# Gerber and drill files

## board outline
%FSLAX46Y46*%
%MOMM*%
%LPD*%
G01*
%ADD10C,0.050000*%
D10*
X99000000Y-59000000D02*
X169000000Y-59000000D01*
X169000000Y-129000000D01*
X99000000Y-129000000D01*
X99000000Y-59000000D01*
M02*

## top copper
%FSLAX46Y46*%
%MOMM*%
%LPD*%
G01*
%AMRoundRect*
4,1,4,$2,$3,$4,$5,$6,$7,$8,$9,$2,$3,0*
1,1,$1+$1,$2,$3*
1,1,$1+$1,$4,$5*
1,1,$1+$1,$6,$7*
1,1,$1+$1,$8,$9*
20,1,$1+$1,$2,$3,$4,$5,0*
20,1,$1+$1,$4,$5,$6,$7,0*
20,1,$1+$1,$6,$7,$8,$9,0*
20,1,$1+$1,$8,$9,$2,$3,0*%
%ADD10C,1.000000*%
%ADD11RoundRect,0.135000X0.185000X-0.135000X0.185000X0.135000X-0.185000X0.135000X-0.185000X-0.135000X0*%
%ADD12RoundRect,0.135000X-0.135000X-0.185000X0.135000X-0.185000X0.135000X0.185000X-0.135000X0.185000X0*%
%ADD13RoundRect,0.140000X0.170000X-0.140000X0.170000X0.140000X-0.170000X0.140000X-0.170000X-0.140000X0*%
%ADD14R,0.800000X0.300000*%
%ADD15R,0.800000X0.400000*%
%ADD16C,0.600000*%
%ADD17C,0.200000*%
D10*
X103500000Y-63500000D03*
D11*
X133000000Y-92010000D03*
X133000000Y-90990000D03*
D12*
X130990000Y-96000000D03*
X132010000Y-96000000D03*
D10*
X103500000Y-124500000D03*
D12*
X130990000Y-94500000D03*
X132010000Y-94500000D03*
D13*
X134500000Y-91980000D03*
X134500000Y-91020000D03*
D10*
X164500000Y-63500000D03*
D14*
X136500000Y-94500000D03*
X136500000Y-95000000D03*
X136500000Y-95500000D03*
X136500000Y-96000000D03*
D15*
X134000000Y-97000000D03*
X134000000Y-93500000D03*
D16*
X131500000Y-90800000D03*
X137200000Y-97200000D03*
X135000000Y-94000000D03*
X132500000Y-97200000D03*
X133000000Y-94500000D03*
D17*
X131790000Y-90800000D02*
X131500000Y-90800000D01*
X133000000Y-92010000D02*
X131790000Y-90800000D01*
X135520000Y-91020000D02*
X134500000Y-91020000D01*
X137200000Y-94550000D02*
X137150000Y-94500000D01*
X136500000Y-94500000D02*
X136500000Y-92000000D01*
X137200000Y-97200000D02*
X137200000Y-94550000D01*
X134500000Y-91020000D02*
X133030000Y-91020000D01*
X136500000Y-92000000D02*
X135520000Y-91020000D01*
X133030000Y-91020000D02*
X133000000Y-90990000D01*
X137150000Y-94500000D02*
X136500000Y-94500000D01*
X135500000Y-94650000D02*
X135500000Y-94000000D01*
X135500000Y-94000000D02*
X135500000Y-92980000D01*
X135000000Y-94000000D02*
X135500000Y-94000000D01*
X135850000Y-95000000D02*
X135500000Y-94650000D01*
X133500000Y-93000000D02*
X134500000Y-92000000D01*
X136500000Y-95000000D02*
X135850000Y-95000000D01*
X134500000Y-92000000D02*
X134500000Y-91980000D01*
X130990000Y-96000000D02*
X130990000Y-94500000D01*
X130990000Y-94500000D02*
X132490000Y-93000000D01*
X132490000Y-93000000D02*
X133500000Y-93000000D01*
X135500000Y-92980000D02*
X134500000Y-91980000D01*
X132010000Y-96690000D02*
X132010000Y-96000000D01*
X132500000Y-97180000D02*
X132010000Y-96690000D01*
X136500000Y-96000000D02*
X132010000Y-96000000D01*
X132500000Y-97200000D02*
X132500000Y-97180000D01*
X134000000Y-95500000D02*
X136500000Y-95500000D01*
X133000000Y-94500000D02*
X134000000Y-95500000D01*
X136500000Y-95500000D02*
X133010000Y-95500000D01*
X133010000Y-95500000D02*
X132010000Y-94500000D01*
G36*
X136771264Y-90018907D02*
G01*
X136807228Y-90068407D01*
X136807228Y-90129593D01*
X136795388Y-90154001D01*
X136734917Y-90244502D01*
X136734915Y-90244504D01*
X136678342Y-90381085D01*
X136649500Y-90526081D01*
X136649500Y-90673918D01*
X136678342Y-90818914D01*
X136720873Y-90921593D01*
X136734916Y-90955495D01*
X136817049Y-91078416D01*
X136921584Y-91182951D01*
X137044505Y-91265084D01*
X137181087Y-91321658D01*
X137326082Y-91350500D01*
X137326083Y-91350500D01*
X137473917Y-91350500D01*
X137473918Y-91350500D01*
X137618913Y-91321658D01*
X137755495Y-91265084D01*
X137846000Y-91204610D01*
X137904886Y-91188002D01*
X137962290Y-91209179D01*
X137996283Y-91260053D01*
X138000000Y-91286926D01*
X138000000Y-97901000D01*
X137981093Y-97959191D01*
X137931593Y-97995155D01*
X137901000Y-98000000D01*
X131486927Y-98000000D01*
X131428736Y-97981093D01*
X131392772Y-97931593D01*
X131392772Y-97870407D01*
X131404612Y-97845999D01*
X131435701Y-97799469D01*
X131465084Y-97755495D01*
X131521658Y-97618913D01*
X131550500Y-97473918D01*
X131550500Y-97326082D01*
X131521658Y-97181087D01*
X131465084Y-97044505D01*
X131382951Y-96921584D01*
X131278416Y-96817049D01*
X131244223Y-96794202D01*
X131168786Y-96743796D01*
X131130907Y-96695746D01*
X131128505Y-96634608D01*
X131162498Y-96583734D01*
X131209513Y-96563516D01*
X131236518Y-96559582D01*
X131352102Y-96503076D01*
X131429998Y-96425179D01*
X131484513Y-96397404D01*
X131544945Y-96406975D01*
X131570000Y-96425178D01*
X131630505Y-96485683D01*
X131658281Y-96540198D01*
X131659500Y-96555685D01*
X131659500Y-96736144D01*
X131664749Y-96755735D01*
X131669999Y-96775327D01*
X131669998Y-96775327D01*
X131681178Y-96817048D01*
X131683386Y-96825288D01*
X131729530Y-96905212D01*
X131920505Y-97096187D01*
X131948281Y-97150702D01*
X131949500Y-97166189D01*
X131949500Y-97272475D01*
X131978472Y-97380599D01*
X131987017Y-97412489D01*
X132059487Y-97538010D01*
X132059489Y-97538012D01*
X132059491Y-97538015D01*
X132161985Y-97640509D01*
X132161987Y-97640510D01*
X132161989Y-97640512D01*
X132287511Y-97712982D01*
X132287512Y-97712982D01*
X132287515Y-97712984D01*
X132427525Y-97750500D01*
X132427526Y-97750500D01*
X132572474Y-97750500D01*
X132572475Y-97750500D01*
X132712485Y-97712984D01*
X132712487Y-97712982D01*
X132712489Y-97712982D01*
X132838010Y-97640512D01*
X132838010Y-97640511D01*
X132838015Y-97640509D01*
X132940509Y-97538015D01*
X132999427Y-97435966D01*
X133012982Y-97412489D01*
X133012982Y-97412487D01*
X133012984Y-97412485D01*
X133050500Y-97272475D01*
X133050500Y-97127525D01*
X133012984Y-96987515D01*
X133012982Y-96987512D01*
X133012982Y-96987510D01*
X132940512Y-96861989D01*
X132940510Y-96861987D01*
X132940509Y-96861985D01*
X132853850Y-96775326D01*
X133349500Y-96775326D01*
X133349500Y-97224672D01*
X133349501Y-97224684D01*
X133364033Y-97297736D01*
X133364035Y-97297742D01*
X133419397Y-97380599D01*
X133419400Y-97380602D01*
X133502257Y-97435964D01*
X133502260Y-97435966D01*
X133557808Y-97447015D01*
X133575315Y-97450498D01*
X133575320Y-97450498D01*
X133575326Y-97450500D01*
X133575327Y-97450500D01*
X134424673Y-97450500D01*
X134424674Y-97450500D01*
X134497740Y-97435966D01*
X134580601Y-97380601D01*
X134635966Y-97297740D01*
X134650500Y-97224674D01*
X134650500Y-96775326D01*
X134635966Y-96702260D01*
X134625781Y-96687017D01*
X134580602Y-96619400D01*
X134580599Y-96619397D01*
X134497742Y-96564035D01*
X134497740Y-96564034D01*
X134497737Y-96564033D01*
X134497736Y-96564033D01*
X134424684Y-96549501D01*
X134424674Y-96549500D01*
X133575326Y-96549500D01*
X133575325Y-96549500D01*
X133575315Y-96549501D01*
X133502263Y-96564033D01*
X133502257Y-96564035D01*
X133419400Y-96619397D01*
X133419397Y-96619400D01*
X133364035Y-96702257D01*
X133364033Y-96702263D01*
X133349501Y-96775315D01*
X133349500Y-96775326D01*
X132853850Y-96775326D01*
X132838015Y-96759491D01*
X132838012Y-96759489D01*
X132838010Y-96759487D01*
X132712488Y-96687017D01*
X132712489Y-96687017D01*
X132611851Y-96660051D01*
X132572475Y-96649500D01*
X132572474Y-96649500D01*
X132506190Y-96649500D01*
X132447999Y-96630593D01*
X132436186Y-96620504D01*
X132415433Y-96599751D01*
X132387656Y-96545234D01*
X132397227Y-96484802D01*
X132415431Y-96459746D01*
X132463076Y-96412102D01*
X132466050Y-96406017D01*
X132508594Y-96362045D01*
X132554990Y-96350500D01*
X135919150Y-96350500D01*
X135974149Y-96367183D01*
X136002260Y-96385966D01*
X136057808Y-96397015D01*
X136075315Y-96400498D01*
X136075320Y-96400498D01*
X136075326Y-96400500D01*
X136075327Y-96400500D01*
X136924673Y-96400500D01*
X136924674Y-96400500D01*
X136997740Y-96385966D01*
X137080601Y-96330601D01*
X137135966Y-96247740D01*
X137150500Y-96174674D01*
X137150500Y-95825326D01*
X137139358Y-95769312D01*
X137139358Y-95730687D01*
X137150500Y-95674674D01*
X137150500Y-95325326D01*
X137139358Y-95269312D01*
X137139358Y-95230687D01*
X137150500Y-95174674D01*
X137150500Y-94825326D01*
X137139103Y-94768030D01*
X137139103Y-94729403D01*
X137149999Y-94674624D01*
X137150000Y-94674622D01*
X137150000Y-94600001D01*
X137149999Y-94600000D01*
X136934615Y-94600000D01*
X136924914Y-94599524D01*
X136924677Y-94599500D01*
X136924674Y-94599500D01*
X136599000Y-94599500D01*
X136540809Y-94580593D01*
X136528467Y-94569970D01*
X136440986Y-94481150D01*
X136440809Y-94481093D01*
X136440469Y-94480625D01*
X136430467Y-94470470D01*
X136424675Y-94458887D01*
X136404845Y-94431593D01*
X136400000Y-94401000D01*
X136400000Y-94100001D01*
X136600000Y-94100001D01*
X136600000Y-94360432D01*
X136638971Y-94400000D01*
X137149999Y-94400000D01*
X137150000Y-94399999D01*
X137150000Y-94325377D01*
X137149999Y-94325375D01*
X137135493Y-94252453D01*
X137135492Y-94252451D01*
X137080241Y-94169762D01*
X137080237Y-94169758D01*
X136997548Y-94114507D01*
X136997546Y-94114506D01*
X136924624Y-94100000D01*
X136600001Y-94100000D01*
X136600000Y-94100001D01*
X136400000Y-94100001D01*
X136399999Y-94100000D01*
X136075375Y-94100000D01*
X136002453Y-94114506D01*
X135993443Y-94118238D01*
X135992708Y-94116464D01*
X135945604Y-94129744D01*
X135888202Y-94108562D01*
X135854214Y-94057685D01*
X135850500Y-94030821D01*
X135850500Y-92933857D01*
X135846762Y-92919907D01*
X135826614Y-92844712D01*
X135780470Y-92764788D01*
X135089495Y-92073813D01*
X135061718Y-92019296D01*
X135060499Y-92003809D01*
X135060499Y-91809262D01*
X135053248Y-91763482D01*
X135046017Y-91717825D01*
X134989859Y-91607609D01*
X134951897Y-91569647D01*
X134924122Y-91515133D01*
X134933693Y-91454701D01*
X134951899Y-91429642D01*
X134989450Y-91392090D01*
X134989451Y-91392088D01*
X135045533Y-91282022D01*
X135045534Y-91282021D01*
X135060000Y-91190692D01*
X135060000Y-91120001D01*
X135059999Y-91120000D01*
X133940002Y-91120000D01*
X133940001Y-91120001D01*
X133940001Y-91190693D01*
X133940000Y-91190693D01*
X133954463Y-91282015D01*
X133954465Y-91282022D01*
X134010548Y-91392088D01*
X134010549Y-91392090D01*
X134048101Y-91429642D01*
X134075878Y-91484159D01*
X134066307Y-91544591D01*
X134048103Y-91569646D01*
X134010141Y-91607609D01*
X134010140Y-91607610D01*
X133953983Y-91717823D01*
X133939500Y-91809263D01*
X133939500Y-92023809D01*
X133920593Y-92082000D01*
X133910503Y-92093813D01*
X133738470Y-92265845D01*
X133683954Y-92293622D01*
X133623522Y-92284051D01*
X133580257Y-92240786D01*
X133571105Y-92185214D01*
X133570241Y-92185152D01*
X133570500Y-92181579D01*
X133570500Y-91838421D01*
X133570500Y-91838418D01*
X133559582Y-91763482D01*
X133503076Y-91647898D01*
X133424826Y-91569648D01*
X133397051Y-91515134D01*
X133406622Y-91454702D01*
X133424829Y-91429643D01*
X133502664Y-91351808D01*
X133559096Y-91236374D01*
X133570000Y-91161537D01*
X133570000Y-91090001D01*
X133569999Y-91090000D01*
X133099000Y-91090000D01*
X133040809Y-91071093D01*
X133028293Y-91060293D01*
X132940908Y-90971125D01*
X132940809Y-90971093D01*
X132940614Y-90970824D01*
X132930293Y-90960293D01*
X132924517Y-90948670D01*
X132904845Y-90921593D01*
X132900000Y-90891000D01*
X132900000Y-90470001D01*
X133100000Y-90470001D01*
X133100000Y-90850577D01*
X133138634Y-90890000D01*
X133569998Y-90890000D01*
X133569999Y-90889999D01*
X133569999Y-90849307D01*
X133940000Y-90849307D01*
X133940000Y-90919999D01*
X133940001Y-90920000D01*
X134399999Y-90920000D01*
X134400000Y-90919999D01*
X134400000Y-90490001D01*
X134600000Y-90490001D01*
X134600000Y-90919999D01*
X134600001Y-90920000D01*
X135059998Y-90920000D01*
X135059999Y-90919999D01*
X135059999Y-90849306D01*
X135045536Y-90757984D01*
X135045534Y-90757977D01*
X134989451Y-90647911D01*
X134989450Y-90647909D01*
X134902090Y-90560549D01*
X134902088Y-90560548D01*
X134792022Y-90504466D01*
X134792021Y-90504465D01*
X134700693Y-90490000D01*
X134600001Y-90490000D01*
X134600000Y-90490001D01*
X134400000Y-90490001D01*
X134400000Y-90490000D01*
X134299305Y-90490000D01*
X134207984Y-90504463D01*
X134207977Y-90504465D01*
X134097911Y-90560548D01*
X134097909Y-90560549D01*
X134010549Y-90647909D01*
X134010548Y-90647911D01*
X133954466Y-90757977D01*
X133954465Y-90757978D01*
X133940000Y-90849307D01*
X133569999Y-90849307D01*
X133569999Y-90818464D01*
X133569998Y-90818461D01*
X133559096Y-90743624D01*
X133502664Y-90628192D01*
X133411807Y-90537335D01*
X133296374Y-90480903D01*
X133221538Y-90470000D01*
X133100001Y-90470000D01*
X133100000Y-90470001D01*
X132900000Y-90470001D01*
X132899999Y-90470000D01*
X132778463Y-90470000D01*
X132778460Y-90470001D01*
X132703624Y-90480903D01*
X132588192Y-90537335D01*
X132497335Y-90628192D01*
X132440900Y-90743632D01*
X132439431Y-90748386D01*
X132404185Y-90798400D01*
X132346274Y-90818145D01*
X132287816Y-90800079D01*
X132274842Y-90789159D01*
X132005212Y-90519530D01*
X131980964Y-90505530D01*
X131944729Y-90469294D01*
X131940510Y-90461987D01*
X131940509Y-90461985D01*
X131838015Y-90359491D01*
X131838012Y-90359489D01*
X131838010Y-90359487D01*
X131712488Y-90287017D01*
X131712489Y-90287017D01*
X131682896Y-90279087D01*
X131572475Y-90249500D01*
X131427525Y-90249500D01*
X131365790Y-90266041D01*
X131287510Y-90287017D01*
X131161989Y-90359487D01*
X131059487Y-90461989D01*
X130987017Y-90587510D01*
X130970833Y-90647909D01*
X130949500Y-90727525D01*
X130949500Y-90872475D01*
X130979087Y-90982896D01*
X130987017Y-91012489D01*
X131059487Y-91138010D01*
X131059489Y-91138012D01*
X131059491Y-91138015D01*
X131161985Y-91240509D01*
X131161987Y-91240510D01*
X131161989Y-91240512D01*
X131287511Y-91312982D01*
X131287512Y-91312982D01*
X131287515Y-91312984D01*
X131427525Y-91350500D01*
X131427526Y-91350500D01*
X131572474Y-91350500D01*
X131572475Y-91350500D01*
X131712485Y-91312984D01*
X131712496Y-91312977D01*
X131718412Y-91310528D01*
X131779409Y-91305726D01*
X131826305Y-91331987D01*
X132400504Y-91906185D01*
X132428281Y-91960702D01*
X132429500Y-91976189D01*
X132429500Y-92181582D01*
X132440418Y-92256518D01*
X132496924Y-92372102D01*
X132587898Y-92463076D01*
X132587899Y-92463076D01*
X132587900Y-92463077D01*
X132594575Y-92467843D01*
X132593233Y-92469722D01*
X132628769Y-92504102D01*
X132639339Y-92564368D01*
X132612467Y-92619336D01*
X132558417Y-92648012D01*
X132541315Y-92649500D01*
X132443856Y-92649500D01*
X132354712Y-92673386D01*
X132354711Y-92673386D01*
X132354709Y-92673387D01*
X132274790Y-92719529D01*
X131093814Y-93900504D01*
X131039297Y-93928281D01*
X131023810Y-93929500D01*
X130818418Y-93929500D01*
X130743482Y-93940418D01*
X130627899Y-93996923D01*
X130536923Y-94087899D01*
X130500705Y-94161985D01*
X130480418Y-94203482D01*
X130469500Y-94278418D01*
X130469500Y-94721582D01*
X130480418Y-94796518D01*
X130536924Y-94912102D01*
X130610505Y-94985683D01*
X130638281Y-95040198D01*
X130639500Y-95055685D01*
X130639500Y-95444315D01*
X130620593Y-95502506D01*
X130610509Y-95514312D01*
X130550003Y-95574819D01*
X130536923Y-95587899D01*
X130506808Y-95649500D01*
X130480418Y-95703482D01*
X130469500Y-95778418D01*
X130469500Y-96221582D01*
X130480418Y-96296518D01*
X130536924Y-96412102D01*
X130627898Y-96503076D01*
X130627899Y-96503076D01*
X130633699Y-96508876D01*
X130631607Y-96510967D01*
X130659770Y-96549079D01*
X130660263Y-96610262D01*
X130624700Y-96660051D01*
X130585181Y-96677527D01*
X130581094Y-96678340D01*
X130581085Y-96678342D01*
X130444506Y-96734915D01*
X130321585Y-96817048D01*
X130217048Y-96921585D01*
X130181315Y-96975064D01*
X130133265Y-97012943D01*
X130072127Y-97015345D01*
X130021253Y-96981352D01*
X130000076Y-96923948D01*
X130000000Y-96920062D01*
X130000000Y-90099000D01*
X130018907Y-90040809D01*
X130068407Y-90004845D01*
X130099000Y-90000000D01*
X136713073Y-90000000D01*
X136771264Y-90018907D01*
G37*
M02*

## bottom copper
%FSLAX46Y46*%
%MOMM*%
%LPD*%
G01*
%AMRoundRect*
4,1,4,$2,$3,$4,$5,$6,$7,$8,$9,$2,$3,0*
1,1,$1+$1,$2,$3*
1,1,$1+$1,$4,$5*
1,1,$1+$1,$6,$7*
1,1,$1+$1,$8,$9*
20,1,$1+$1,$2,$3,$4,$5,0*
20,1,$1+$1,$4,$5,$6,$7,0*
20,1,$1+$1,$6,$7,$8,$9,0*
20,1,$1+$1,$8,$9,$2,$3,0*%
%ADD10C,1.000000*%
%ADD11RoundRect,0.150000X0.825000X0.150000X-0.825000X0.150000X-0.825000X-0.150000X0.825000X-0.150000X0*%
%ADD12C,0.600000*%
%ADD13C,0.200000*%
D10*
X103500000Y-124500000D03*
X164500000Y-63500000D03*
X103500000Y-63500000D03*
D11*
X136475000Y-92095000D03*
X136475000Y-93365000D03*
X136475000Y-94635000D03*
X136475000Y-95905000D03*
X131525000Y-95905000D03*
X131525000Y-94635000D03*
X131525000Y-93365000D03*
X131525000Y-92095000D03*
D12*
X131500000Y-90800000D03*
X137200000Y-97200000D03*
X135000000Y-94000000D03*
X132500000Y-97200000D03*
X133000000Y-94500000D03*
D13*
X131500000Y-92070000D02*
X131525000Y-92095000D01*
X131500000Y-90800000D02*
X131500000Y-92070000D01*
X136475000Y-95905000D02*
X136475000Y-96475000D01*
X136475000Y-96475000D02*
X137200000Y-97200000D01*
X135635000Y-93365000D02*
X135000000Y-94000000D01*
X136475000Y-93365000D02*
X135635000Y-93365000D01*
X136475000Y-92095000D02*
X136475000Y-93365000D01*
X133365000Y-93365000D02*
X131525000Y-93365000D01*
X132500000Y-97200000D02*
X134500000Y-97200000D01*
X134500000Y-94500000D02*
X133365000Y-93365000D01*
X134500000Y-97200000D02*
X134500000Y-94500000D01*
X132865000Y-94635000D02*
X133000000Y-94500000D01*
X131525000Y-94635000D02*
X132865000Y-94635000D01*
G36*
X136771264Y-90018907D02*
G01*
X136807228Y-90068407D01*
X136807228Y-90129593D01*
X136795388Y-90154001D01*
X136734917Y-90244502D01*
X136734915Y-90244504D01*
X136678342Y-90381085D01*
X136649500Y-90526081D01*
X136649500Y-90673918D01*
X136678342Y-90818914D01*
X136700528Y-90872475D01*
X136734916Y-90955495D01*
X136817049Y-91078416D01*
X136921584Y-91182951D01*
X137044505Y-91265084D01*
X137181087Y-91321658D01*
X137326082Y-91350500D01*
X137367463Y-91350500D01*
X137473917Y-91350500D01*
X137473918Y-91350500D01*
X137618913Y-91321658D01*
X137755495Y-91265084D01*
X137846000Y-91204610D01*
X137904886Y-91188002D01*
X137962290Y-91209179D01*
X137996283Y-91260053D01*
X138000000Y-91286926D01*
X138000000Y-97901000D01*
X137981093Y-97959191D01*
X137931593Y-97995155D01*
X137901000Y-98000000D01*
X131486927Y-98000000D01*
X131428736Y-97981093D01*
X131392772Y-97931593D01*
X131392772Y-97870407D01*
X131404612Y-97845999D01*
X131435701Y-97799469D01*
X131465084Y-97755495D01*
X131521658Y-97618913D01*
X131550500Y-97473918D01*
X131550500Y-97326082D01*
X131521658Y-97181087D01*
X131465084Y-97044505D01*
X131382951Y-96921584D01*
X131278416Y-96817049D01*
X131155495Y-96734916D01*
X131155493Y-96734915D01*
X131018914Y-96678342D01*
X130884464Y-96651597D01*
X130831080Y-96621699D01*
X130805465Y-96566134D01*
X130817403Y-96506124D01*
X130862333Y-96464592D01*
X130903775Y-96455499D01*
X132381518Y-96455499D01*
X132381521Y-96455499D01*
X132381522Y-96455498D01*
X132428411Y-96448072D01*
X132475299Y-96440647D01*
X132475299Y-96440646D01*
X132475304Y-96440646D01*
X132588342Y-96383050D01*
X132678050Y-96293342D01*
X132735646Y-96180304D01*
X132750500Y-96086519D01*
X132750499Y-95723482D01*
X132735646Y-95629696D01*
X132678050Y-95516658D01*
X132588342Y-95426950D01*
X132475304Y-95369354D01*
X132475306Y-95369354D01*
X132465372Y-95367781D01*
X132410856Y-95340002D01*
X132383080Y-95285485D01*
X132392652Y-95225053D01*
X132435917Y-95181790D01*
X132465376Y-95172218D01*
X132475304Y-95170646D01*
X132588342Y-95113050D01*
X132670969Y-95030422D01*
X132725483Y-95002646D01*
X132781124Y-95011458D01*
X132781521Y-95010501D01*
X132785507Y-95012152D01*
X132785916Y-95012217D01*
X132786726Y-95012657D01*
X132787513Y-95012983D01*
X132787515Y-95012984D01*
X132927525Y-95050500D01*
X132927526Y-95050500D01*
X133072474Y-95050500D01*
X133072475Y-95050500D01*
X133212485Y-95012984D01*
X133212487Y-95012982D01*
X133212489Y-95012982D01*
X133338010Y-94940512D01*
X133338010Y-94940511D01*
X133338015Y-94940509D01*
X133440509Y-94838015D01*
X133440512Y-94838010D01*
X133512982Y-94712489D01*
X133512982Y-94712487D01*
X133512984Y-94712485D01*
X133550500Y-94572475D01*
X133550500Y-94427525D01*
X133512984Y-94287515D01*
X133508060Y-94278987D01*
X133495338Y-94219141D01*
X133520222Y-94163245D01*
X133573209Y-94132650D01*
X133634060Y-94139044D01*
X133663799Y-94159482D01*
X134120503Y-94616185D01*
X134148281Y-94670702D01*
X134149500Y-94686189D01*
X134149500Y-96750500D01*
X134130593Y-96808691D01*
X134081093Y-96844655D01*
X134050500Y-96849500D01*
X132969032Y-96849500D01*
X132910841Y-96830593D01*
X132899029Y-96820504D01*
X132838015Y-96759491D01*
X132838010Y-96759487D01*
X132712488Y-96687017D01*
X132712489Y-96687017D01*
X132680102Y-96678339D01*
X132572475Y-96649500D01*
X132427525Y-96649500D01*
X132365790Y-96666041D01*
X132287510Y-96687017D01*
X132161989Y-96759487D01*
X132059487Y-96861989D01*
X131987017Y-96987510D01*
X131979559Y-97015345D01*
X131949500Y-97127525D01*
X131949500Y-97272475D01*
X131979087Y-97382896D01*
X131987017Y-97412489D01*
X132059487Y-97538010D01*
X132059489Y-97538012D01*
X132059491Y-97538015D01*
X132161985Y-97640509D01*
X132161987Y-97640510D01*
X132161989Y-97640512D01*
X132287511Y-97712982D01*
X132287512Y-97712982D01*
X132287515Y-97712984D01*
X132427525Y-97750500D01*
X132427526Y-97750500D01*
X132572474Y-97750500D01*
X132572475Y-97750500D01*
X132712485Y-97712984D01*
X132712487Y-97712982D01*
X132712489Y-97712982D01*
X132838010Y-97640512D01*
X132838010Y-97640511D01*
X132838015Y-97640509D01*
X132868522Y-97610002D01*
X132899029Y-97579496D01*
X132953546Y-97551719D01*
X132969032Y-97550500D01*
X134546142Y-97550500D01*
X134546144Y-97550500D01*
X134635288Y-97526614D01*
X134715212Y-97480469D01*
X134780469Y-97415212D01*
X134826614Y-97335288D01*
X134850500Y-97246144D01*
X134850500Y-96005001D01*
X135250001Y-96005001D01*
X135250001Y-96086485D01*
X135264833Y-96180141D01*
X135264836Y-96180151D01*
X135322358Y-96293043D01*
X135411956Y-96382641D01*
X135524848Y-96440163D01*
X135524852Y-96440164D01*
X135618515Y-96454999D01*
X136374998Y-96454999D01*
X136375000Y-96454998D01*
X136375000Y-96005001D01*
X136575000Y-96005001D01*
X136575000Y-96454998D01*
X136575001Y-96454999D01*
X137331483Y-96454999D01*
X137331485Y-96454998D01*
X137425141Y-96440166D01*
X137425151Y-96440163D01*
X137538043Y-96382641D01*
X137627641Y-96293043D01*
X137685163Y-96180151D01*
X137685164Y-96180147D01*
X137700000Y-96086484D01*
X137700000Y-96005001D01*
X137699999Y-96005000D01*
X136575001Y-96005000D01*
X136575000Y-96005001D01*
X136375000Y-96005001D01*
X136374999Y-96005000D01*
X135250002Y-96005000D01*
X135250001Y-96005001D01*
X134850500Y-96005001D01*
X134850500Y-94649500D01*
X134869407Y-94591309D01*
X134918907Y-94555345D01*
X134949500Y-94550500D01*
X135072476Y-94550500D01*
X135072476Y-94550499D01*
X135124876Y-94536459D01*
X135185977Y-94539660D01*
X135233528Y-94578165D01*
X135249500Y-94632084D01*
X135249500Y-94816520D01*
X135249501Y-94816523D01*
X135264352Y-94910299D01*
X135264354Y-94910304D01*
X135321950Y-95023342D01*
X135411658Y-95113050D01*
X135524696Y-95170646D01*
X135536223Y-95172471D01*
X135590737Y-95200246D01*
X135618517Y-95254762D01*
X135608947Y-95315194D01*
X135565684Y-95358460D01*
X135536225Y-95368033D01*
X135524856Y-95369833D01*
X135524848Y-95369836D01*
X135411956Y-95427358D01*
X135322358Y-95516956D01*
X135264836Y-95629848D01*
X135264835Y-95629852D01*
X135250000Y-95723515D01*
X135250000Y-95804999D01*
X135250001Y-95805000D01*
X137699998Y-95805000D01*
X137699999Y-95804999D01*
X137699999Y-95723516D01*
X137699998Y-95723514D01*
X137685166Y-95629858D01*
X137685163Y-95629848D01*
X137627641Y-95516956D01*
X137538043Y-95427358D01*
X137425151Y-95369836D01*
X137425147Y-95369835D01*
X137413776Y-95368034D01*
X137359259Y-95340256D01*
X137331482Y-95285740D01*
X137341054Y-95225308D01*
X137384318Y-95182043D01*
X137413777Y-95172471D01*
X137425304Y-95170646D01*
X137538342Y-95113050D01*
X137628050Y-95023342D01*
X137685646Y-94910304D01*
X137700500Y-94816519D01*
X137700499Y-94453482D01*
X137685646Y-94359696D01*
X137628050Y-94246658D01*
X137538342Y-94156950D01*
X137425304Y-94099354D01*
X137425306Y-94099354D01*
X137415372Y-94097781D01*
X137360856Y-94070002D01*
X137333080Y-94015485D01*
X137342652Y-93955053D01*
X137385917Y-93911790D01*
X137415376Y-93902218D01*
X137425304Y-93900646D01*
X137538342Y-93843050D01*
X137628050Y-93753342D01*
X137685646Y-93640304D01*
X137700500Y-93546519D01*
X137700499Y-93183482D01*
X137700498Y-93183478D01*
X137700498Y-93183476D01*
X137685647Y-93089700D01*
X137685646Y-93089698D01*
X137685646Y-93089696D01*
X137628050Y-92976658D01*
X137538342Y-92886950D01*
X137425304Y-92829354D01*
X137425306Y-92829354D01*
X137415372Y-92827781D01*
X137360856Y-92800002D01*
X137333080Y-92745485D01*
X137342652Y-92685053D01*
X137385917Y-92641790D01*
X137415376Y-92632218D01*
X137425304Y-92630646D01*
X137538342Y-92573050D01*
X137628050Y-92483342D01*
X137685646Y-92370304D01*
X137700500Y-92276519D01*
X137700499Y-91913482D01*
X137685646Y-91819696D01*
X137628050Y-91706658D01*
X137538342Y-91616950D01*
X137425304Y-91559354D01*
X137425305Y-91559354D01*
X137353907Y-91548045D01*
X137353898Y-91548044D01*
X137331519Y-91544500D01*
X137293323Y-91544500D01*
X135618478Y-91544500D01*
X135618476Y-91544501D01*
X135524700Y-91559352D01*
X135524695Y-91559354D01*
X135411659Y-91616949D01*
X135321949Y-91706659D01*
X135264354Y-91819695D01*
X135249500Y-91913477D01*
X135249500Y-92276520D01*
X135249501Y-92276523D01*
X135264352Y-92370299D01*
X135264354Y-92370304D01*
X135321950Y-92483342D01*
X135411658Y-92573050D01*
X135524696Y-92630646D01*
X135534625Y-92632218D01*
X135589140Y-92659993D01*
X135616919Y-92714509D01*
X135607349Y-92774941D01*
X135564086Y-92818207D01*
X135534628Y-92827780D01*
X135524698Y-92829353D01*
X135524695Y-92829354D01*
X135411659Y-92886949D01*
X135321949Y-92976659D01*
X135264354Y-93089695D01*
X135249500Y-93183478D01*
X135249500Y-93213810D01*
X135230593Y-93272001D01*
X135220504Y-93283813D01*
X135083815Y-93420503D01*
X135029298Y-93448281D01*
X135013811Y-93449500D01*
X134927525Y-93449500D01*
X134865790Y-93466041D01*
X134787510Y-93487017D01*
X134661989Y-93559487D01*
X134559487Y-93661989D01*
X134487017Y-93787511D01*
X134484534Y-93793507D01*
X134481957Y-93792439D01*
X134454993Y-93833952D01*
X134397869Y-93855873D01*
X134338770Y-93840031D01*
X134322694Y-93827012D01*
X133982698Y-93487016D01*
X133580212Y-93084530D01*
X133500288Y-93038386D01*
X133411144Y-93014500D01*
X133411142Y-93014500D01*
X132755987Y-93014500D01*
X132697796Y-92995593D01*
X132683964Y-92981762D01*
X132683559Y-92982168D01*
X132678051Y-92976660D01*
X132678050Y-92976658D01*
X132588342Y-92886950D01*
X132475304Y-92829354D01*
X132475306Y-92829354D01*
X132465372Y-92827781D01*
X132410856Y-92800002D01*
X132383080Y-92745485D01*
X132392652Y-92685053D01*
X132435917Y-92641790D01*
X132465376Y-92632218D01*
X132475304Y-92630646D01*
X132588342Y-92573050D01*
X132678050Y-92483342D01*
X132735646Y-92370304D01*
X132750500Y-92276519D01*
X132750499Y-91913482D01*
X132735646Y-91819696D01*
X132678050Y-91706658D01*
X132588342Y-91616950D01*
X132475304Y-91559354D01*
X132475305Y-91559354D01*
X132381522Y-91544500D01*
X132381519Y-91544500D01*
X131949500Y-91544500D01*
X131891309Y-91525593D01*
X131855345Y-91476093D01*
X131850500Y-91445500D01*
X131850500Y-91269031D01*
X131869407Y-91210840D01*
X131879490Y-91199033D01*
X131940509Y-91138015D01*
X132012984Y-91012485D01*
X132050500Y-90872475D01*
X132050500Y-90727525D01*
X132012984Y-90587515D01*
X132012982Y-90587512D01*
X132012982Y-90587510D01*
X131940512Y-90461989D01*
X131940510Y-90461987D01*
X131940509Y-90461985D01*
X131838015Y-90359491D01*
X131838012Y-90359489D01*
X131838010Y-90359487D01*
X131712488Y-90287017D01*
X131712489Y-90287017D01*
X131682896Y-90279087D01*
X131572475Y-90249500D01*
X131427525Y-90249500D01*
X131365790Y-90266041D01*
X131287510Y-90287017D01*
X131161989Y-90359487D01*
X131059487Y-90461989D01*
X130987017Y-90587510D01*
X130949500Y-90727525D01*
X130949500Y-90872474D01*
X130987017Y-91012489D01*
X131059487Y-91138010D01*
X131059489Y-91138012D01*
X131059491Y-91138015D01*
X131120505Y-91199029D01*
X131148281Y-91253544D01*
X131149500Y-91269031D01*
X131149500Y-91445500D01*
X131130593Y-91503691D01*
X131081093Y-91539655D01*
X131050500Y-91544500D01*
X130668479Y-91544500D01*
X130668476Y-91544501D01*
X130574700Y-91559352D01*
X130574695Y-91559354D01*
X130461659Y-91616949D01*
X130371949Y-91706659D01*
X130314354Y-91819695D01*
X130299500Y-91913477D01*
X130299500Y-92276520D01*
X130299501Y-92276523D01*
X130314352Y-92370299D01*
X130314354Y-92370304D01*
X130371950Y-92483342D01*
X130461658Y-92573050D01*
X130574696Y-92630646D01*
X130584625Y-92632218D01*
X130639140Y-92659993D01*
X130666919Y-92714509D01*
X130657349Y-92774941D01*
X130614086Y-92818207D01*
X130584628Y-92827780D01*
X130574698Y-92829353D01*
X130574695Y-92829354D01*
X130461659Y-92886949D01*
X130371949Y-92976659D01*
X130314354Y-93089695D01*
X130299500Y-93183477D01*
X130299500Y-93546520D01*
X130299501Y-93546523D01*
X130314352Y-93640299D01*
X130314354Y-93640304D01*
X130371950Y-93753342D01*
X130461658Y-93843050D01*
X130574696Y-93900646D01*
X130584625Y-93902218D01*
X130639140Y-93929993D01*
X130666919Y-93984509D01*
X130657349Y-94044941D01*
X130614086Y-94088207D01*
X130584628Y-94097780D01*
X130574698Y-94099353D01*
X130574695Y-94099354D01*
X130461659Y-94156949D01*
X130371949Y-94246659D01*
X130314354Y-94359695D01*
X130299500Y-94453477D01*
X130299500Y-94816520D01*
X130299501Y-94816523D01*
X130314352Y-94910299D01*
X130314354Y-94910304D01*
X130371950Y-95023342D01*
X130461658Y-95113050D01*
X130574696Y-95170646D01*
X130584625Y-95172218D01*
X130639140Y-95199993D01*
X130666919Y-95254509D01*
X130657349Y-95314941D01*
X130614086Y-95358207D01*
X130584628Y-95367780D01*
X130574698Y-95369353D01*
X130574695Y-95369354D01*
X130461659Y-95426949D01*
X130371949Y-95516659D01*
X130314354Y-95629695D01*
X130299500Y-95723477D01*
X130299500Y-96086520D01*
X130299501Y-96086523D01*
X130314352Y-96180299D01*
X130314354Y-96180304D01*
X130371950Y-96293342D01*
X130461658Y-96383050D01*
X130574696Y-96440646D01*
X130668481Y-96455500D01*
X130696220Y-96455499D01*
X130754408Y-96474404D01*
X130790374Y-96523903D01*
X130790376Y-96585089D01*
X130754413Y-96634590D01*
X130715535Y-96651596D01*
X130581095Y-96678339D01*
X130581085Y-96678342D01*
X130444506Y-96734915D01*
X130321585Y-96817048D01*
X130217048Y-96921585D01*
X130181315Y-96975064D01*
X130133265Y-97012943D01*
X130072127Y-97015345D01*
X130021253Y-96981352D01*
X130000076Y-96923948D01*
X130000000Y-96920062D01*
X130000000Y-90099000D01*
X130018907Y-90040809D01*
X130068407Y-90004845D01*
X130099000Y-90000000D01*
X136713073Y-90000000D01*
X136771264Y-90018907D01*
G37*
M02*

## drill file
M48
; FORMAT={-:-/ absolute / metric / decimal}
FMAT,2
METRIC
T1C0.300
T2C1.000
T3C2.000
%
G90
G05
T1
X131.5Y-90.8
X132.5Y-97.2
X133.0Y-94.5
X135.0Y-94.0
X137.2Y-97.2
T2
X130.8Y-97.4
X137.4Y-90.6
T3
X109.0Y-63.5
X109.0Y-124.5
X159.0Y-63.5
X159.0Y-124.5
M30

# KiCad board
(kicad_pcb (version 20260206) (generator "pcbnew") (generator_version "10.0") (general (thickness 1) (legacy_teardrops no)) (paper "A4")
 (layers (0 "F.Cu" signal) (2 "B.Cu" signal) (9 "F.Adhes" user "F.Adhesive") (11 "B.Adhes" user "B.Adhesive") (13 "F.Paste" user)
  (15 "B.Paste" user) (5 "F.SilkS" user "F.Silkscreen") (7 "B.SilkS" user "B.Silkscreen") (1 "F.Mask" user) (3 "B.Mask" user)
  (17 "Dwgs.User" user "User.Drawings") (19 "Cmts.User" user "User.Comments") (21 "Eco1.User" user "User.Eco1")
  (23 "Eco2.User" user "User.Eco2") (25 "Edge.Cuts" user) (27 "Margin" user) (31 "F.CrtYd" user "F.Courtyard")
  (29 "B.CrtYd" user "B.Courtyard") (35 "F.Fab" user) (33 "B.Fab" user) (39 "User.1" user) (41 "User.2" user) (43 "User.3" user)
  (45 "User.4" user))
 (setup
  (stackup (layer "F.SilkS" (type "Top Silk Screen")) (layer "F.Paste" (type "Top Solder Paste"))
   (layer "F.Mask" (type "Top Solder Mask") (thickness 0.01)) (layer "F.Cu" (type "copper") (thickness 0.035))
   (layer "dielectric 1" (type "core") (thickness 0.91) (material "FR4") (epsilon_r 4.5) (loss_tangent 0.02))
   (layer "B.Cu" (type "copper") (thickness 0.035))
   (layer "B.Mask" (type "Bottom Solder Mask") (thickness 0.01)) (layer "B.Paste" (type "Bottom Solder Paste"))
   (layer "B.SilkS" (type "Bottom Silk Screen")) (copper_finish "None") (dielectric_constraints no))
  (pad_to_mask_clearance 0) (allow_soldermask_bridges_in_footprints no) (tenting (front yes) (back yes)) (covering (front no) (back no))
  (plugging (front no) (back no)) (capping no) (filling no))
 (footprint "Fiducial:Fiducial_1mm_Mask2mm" (layer "F.Cu") (at 103.5 63.5)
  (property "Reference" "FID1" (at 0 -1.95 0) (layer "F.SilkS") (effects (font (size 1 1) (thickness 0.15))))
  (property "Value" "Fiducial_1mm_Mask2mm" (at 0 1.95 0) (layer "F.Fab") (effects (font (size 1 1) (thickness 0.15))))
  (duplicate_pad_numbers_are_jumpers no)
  (pad "" smd circle (at 0 0) (size 1 1) (layers "F.Cu" "F.Mask") (solder_mask_margin 0.5) (clearance 0.6)))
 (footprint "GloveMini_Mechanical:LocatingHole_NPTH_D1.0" (layer "F.Cu") (at 137.4 90.6)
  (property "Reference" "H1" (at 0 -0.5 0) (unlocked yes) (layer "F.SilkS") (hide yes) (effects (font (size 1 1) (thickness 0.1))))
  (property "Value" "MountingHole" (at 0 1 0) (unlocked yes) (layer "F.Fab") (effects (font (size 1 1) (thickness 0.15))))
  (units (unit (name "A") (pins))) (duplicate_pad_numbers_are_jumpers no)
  (pad "" np_thru_hole circle (at 0 0) (size 1 1) (drill 1) (layers "*.Cu" "*.Mask")))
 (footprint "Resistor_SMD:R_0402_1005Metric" (layer "F.Cu") (at 133 91.5 90)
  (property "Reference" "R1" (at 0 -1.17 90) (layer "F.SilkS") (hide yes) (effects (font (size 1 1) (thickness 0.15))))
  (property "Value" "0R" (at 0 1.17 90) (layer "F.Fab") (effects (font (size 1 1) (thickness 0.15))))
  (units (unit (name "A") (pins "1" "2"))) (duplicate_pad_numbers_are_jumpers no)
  (pad "1" smd roundrect (at -0.51 0 90) (size 0.54 0.64) (layers "F.Cu" "F.Mask" "F.Paste") (roundrect_rratio 0.25) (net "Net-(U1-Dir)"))
  (pad "2" smd roundrect (at 0.51 0 90) (size 0.54 0.64) (layers "F.Cu" "F.Mask" "F.Paste") (roundrect_rratio 0.25) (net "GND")))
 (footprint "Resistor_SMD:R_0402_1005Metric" (layer "F.Cu") (at 131.5 96)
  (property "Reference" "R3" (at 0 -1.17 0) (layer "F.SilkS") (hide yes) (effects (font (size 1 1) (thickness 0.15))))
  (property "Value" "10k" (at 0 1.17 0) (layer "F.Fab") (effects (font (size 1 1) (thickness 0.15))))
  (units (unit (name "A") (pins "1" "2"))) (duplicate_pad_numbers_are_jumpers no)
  (pad "1" smd roundrect (at -0.51 0) (size 0.54 0.64) (layers "F.Cu" "F.Mask" "F.Paste") (roundrect_rratio 0.25) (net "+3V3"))
  (pad "2" smd roundrect (at 0.51 0) (size 0.54 0.64) (layers "F.Cu" "F.Mask" "F.Paste") (roundrect_rratio 0.25) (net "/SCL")))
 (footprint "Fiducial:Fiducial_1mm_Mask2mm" (layer "F.Cu") (at 103.5 124.5)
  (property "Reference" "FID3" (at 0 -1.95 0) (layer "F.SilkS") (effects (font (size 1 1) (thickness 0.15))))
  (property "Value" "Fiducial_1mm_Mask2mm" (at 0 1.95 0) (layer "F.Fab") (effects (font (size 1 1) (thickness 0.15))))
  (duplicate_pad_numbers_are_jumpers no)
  (pad "" smd circle (at 0 0) (size 1 1) (layers "F.Cu" "F.Mask") (solder_mask_margin 0.5) (clearance 0.6)))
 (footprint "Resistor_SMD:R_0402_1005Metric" (layer "F.Cu") (at 131.5 94.5)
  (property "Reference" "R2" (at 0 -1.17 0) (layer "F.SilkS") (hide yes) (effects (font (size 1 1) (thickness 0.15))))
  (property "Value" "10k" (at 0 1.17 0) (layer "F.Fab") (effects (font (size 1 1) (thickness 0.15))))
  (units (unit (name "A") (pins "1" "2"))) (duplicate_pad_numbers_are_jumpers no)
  (pad "1" smd roundrect (at -0.51 0) (size 0.54 0.64) (layers "F.Cu" "F.Mask" "F.Paste") (roundrect_rratio 0.25) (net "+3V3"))
  (pad "2" smd roundrect (at 0.51 0) (size 0.54 0.64) (layers "F.Cu" "F.Mask" "F.Paste") (roundrect_rratio 0.25) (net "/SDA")))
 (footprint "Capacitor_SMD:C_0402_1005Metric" (layer "F.Cu") (at 134.5 91.5 90)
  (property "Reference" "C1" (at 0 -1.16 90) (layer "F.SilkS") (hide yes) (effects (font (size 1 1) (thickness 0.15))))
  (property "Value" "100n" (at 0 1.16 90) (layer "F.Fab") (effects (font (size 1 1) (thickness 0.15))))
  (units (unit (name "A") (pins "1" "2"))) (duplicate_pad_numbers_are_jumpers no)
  (pad "1" smd roundrect (at -0.48 0 90) (size 0.56 0.62) (layers "F.Cu" "F.Mask" "F.Paste") (roundrect_rratio 0.25) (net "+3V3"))
  (pad "2" smd roundrect (at 0.48 0 90) (size 0.56 0.62) (layers "F.Cu" "F.Mask" "F.Paste") (roundrect_rratio 0.25) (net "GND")))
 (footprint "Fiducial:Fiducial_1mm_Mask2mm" (layer "F.Cu") (at 164.5 63.5)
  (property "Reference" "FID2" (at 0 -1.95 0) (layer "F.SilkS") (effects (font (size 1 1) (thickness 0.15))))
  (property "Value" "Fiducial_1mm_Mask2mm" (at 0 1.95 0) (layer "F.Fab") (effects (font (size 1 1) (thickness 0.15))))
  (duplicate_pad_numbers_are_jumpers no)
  (pad "" smd circle (at 0 0) (size 1 1) (layers "F.Cu" "F.Mask") (solder_mask_margin 0.5) (clearance 0.6)))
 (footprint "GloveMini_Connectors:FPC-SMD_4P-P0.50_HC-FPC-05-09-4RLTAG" (layer "F.Cu") (at 135.25 95.25 90)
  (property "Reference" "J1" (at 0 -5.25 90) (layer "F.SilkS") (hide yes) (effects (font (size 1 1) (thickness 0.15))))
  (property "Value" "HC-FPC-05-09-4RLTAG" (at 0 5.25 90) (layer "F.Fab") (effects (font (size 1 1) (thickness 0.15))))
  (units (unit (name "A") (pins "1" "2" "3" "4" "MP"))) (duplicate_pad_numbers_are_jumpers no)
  (pad "1" smd rect (at 0.75 1.25 270) (size 0.3 0.8) (layers "F.Cu" "F.Mask" "F.Paste") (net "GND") (solder_paste_margin 0.005)
   (solder_paste_margin_ratio -0.1))
  (pad "2" smd rect (at 0.25 1.25 270) (size 0.3 0.8) (layers "F.Cu" "F.Mask" "F.Paste") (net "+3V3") (solder_paste_margin 0.005)
   (solder_paste_margin_ratio -0.1))
  (pad "3" smd rect (at -0.25 1.25 270) (size 0.3 0.8) (layers "F.Cu" "F.Mask" "F.Paste") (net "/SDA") (solder_paste_margin 0.005)
   (solder_paste_margin_ratio -0.1))
  (pad "4" smd rect (at -0.75 1.25 270) (size 0.3 0.8) (layers "F.Cu" "F.Mask" "F.Paste") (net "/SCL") (solder_paste_margin 0.005)
   (solder_paste_margin_ratio -0.1))
  (pad "MP" smd rect (at -1.75 -1.25 270) (size 0.4 0.8) (layers "F.Cu" "F.Mask" "F.Paste") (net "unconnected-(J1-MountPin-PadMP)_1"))
  (pad "MP" smd rect (at 1.75 -1.25 270) (size 0.4 0.8) (layers "F.Cu" "F.Mask" "F.Paste") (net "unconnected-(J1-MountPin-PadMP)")))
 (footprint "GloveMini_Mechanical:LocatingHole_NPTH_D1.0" (layer "F.Cu") (at 130.8 97.4)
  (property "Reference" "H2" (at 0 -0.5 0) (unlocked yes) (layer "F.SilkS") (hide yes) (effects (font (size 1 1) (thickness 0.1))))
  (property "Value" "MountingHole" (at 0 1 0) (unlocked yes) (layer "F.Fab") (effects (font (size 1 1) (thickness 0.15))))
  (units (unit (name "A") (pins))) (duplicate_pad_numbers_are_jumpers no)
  (pad "" np_thru_hole circle (at 0 0) (size 1 1) (drill 1) (layers "*.Cu" "*.Mask")))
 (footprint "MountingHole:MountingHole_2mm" (layer "F.Cu") (at 109 124.5)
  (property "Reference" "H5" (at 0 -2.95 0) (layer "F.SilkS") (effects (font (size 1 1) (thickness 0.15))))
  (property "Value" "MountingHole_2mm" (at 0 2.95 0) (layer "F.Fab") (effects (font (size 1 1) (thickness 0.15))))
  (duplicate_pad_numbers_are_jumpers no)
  (pad "" np_thru_hole circle (at 0 0) (size 2 2) (drill 2) (layers "*.Cu" "*.Mask")))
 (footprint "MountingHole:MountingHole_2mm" (layer "F.Cu") (at 159 63.5)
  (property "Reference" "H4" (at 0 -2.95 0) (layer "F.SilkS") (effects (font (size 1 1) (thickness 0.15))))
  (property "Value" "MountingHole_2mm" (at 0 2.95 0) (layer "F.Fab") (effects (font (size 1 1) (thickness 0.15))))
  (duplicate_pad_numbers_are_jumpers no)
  (pad "" np_thru_hole circle (at 0 0) (size 2 2) (drill 2) (layers "*.Cu" "*.Mask")))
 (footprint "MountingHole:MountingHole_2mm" (layer "F.Cu") (at 159 124.5)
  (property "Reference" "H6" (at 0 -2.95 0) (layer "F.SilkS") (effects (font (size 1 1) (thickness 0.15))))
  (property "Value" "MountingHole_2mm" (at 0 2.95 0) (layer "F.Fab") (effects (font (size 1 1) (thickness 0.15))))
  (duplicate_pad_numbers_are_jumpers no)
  (pad "" np_thru_hole circle (at 0 0) (size 2 2) (drill 2) (layers "*.Cu" "*.Mask")))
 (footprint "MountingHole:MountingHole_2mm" (layer "F.Cu") (at 109 63.5)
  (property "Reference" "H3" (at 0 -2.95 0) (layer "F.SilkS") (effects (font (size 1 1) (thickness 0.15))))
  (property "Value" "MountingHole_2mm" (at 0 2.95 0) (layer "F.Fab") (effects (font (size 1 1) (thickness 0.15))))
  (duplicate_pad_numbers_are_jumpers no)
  (pad "" np_thru_hole circle (at 0 0) (size 2 2) (drill 2) (layers "*.Cu" "*.Mask")))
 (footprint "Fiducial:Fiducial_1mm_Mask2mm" (layer "B.Cu") (at 103.5 124.5 180)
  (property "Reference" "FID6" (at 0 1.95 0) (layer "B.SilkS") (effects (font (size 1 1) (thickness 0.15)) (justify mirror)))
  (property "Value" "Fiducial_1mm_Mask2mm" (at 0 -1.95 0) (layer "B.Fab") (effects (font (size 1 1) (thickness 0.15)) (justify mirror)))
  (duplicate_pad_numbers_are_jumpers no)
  (pad "" smd circle (at 0 0 180) (size 1 1) (layers "B.Cu" "B.Mask") (solder_mask_margin 0.5) (clearance 0.6)))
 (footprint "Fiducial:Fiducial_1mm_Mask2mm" (layer "B.Cu") (at 164.5 63.5 180)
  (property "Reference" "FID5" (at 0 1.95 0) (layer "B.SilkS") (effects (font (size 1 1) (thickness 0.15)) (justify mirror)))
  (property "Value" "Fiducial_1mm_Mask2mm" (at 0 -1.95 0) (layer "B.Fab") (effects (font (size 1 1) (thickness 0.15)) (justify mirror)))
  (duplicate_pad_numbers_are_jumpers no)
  (pad "" smd circle (at 0 0 180) (size 1 1) (layers "B.Cu" "B.Mask") (solder_mask_margin 0.5) (clearance 0.6)))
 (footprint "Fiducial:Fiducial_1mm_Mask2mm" (layer "B.Cu") (at 103.5 63.5 180)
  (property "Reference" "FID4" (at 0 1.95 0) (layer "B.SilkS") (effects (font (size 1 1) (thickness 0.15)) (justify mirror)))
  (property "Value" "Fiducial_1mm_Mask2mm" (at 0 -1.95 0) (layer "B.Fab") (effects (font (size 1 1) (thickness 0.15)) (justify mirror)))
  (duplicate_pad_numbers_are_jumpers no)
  (pad "" smd circle (at 0 0 180) (size 1 1) (layers "B.Cu" "B.Mask") (solder_mask_margin 0.5) (clearance 0.6)))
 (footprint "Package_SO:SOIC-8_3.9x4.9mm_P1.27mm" (layer "B.Cu") (at 134 94 180)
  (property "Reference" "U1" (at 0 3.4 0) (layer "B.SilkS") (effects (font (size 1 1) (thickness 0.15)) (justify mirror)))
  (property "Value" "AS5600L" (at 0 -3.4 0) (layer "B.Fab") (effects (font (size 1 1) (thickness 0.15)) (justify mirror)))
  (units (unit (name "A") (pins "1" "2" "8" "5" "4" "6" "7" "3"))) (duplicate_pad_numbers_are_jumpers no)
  (pad "1" smd roundrect (at -2.475 1.905 180) (size 1.95 0.6) (layers "B.Cu" "B.Mask" "B.Paste") (roundrect_rratio 0.25) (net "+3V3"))
  (pad "2" smd roundrect (at -2.475 0.635 180) (size 1.95 0.6) (layers "B.Cu" "B.Mask" "B.Paste") (roundrect_rratio 0.25) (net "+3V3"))
  (pad "3" smd roundrect (at -2.475 -0.635 180) (size 1.95 0.6) (layers "B.Cu" "B.Mask" "B.Paste") (roundrect_rratio 0.25)
   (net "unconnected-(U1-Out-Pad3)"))
  (pad "4" smd roundrect (at -2.475 -1.905 180) (size 1.95 0.6) (layers "B.Cu" "B.Mask" "B.Paste") (roundrect_rratio 0.25) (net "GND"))
  (pad "5" smd roundrect (at 2.475 -1.905 180) (size 1.95 0.6) (layers "B.Cu" "B.Mask" "B.Paste") (roundrect_rratio 0.25)
   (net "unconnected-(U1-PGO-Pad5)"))
  (pad "6" smd roundrect (at 2.475 -0.635 180) (size 1.95 0.6) (layers "B.Cu" "B.Mask" "B.Paste") (roundrect_rratio 0.25) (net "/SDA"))
  (pad "7" smd roundrect (at 2.475 0.635 180) (size 1.95 0.6) (layers "B.Cu" "B.Mask" "B.Paste") (roundrect_rratio 0.25) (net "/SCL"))
  (pad "8" smd roundrect (at 2.475 1.905 180) (size 1.95 0.6) (layers "B.Cu" "B.Mask" "B.Paste") (roundrect_rratio 0.25)
   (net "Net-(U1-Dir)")))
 (gr_rect (start 99 59) (end 169 129) (stroke (width 0.05) (type solid)) (fill no) (layer "Edge.Cuts"))
 (segment (start 131.79 90.8) (end 131.5 90.8) (width 0.2) (layer "F.Cu") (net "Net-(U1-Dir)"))
 (segment (start 133 92.01) (end 131.79 90.8) (width 0.2) (layer "F.Cu") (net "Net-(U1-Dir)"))
 (via (at 131.5 90.8) (size 0.6) (drill 0.3) (layers "F.Cu" "B.Cu") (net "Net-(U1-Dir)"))
 (segment (start 131.5 92.07) (end 131.525 92.095) (width 0.2) (layer "B.Cu") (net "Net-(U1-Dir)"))
 (segment (start 131.5 90.8) (end 131.5 92.07) (width 0.2) (layer "B.Cu") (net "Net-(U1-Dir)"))
 (segment (start 135.52 91.02) (end 134.5 91.02) (width 0.2) (layer "F.Cu") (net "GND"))
 (segment (start 137.2 94.55) (end 137.15 94.5) (width 0.2) (layer "F.Cu") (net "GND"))
 (segment (start 136.5 94.5) (end 136.5 92) (width 0.2) (layer "F.Cu") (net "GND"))
 (segment (start 137.2 97.2) (end 137.2 94.55) (width 0.2) (layer "F.Cu") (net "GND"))
 (segment (start 134.5 91.02) (end 133.03 91.02) (width 0.2) (layer "F.Cu") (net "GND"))
 (segment (start 136.5 92) (end 135.52 91.02) (width 0.2) (layer "F.Cu") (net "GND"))
 (segment (start 133.03 91.02) (end 133 90.99) (width 0.2) (layer "F.Cu") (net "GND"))
 (segment (start 137.15 94.5) (end 136.5 94.5) (width 0.2) (layer "F.Cu") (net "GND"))
 (via (at 137.2 97.2) (size 0.6) (drill 0.3) (layers "F.Cu" "B.Cu") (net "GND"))
 (segment (start 136.475 95.905) (end 136.475 96.475) (width 0.2) (layer "B.Cu") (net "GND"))
 (segment (start 136.475 96.475) (end 137.2 97.2) (width 0.2) (layer "B.Cu") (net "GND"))
 (segment (start 135.5 94.65) (end 135.5 94) (width 0.2) (layer "F.Cu") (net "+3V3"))
 (segment (start 135.5 94) (end 135.5 92.98) (width 0.2) (layer "F.Cu") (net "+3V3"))
 (segment (start 135 94) (end 135.5 94) (width 0.2) (layer "F.Cu") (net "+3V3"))
 (segment (start 135.85 95) (end 135.5 94.65) (width 0.2) (layer "F.Cu") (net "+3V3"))
 (segment (start 133.5 93) (end 134.5 92) (width 0.2) (layer "F.Cu") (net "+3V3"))
 (segment (start 136.5 95) (end 135.85 95) (width 0.2) (layer "F.Cu") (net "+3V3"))
 (segment (start 134.5 92) (end 134.5 91.98) (width 0.2) (layer "F.Cu") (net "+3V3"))
 (segment (start 130.99 96) (end 130.99 94.5) (width 0.2) (layer "F.Cu") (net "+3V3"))
 (segment (start 130.99 94.5) (end 132.49 93) (width 0.2) (layer "F.Cu") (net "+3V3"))
 (segment (start 132.49 93) (end 133.5 93) (width 0.2) (layer "F.Cu") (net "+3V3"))
 (segment (start 135.5 92.98) (end 134.5 91.98) (width 0.2) (layer "F.Cu") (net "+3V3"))
 (via (at 135 94) (size 0.6) (drill 0.3) (layers "F.Cu" "B.Cu") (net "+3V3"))
 (segment (start 135.635 93.365) (end 135 94) (width 0.2) (layer "B.Cu") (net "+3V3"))
 (segment (start 136.475 93.365) (end 135.635 93.365) (width 0.2) (layer "B.Cu") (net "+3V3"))
 (segment (start 136.475 92.095) (end 136.475 93.365) (width 0.2) (layer "B.Cu") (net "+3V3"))
 (segment (start 132.01 96.69) (end 132.01 96) (width 0.2) (layer "F.Cu") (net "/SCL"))
 (segment (start 132.5 97.18) (end 132.01 96.69) (width 0.2) (layer "F.Cu") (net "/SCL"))
 (segment (start 136.5 96) (end 132.01 96) (width 0.2) (layer "F.Cu") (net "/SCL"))
 (segment (start 132.5 97.2) (end 132.5 97.18) (width 0.2) (layer "F.Cu") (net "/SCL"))
 (via (at 132.5 97.2) (size 0.6) (drill 0.3) (layers "F.Cu" "B.Cu") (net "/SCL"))
 (segment (start 133.365 93.365) (end 131.525 93.365) (width 0.2) (layer "B.Cu") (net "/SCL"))
 (segment (start 132.5 97.2) (end 134.5 97.2) (width 0.2) (layer "B.Cu") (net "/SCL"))
 (segment (start 134.5 94.5) (end 133.365 93.365) (width 0.2) (layer "B.Cu") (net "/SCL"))
 (segment (start 134.5 97.2) (end 134.5 94.5) (width 0.2) (layer "B.Cu") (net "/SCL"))
 (segment (start 134 95.5) (end 136.5 95.5) (width 0.2) (layer "F.Cu") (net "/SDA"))
 (segment (start 133 94.5) (end 134 95.5) (width 0.2) (layer "F.Cu") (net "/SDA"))
 (segment (start 136.5 95.5) (end 133.01 95.5) (width 0.2) (layer "F.Cu") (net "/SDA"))
 (segment (start 133.01 95.5) (end 132.01 94.5) (width 0.2) (layer "F.Cu") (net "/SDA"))
 (via (at 133 94.5) (size 0.6) (drill 0.3) (layers "F.Cu" "B.Cu") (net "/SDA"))
 (segment (start 132.865 94.635) (end 133 94.5) (width 0.2) (layer "B.Cu") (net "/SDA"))
 (segment (start 131.525 94.635) (end 132.865 94.635) (width 0.2) (layer "B.Cu") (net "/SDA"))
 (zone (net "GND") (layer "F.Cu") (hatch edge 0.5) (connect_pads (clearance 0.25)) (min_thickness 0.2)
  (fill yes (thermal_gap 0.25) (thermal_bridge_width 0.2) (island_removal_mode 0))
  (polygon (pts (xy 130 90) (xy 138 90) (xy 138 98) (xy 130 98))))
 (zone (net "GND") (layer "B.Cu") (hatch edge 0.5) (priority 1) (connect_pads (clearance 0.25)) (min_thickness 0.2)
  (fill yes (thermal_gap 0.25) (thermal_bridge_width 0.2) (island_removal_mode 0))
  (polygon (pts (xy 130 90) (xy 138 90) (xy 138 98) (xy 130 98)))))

